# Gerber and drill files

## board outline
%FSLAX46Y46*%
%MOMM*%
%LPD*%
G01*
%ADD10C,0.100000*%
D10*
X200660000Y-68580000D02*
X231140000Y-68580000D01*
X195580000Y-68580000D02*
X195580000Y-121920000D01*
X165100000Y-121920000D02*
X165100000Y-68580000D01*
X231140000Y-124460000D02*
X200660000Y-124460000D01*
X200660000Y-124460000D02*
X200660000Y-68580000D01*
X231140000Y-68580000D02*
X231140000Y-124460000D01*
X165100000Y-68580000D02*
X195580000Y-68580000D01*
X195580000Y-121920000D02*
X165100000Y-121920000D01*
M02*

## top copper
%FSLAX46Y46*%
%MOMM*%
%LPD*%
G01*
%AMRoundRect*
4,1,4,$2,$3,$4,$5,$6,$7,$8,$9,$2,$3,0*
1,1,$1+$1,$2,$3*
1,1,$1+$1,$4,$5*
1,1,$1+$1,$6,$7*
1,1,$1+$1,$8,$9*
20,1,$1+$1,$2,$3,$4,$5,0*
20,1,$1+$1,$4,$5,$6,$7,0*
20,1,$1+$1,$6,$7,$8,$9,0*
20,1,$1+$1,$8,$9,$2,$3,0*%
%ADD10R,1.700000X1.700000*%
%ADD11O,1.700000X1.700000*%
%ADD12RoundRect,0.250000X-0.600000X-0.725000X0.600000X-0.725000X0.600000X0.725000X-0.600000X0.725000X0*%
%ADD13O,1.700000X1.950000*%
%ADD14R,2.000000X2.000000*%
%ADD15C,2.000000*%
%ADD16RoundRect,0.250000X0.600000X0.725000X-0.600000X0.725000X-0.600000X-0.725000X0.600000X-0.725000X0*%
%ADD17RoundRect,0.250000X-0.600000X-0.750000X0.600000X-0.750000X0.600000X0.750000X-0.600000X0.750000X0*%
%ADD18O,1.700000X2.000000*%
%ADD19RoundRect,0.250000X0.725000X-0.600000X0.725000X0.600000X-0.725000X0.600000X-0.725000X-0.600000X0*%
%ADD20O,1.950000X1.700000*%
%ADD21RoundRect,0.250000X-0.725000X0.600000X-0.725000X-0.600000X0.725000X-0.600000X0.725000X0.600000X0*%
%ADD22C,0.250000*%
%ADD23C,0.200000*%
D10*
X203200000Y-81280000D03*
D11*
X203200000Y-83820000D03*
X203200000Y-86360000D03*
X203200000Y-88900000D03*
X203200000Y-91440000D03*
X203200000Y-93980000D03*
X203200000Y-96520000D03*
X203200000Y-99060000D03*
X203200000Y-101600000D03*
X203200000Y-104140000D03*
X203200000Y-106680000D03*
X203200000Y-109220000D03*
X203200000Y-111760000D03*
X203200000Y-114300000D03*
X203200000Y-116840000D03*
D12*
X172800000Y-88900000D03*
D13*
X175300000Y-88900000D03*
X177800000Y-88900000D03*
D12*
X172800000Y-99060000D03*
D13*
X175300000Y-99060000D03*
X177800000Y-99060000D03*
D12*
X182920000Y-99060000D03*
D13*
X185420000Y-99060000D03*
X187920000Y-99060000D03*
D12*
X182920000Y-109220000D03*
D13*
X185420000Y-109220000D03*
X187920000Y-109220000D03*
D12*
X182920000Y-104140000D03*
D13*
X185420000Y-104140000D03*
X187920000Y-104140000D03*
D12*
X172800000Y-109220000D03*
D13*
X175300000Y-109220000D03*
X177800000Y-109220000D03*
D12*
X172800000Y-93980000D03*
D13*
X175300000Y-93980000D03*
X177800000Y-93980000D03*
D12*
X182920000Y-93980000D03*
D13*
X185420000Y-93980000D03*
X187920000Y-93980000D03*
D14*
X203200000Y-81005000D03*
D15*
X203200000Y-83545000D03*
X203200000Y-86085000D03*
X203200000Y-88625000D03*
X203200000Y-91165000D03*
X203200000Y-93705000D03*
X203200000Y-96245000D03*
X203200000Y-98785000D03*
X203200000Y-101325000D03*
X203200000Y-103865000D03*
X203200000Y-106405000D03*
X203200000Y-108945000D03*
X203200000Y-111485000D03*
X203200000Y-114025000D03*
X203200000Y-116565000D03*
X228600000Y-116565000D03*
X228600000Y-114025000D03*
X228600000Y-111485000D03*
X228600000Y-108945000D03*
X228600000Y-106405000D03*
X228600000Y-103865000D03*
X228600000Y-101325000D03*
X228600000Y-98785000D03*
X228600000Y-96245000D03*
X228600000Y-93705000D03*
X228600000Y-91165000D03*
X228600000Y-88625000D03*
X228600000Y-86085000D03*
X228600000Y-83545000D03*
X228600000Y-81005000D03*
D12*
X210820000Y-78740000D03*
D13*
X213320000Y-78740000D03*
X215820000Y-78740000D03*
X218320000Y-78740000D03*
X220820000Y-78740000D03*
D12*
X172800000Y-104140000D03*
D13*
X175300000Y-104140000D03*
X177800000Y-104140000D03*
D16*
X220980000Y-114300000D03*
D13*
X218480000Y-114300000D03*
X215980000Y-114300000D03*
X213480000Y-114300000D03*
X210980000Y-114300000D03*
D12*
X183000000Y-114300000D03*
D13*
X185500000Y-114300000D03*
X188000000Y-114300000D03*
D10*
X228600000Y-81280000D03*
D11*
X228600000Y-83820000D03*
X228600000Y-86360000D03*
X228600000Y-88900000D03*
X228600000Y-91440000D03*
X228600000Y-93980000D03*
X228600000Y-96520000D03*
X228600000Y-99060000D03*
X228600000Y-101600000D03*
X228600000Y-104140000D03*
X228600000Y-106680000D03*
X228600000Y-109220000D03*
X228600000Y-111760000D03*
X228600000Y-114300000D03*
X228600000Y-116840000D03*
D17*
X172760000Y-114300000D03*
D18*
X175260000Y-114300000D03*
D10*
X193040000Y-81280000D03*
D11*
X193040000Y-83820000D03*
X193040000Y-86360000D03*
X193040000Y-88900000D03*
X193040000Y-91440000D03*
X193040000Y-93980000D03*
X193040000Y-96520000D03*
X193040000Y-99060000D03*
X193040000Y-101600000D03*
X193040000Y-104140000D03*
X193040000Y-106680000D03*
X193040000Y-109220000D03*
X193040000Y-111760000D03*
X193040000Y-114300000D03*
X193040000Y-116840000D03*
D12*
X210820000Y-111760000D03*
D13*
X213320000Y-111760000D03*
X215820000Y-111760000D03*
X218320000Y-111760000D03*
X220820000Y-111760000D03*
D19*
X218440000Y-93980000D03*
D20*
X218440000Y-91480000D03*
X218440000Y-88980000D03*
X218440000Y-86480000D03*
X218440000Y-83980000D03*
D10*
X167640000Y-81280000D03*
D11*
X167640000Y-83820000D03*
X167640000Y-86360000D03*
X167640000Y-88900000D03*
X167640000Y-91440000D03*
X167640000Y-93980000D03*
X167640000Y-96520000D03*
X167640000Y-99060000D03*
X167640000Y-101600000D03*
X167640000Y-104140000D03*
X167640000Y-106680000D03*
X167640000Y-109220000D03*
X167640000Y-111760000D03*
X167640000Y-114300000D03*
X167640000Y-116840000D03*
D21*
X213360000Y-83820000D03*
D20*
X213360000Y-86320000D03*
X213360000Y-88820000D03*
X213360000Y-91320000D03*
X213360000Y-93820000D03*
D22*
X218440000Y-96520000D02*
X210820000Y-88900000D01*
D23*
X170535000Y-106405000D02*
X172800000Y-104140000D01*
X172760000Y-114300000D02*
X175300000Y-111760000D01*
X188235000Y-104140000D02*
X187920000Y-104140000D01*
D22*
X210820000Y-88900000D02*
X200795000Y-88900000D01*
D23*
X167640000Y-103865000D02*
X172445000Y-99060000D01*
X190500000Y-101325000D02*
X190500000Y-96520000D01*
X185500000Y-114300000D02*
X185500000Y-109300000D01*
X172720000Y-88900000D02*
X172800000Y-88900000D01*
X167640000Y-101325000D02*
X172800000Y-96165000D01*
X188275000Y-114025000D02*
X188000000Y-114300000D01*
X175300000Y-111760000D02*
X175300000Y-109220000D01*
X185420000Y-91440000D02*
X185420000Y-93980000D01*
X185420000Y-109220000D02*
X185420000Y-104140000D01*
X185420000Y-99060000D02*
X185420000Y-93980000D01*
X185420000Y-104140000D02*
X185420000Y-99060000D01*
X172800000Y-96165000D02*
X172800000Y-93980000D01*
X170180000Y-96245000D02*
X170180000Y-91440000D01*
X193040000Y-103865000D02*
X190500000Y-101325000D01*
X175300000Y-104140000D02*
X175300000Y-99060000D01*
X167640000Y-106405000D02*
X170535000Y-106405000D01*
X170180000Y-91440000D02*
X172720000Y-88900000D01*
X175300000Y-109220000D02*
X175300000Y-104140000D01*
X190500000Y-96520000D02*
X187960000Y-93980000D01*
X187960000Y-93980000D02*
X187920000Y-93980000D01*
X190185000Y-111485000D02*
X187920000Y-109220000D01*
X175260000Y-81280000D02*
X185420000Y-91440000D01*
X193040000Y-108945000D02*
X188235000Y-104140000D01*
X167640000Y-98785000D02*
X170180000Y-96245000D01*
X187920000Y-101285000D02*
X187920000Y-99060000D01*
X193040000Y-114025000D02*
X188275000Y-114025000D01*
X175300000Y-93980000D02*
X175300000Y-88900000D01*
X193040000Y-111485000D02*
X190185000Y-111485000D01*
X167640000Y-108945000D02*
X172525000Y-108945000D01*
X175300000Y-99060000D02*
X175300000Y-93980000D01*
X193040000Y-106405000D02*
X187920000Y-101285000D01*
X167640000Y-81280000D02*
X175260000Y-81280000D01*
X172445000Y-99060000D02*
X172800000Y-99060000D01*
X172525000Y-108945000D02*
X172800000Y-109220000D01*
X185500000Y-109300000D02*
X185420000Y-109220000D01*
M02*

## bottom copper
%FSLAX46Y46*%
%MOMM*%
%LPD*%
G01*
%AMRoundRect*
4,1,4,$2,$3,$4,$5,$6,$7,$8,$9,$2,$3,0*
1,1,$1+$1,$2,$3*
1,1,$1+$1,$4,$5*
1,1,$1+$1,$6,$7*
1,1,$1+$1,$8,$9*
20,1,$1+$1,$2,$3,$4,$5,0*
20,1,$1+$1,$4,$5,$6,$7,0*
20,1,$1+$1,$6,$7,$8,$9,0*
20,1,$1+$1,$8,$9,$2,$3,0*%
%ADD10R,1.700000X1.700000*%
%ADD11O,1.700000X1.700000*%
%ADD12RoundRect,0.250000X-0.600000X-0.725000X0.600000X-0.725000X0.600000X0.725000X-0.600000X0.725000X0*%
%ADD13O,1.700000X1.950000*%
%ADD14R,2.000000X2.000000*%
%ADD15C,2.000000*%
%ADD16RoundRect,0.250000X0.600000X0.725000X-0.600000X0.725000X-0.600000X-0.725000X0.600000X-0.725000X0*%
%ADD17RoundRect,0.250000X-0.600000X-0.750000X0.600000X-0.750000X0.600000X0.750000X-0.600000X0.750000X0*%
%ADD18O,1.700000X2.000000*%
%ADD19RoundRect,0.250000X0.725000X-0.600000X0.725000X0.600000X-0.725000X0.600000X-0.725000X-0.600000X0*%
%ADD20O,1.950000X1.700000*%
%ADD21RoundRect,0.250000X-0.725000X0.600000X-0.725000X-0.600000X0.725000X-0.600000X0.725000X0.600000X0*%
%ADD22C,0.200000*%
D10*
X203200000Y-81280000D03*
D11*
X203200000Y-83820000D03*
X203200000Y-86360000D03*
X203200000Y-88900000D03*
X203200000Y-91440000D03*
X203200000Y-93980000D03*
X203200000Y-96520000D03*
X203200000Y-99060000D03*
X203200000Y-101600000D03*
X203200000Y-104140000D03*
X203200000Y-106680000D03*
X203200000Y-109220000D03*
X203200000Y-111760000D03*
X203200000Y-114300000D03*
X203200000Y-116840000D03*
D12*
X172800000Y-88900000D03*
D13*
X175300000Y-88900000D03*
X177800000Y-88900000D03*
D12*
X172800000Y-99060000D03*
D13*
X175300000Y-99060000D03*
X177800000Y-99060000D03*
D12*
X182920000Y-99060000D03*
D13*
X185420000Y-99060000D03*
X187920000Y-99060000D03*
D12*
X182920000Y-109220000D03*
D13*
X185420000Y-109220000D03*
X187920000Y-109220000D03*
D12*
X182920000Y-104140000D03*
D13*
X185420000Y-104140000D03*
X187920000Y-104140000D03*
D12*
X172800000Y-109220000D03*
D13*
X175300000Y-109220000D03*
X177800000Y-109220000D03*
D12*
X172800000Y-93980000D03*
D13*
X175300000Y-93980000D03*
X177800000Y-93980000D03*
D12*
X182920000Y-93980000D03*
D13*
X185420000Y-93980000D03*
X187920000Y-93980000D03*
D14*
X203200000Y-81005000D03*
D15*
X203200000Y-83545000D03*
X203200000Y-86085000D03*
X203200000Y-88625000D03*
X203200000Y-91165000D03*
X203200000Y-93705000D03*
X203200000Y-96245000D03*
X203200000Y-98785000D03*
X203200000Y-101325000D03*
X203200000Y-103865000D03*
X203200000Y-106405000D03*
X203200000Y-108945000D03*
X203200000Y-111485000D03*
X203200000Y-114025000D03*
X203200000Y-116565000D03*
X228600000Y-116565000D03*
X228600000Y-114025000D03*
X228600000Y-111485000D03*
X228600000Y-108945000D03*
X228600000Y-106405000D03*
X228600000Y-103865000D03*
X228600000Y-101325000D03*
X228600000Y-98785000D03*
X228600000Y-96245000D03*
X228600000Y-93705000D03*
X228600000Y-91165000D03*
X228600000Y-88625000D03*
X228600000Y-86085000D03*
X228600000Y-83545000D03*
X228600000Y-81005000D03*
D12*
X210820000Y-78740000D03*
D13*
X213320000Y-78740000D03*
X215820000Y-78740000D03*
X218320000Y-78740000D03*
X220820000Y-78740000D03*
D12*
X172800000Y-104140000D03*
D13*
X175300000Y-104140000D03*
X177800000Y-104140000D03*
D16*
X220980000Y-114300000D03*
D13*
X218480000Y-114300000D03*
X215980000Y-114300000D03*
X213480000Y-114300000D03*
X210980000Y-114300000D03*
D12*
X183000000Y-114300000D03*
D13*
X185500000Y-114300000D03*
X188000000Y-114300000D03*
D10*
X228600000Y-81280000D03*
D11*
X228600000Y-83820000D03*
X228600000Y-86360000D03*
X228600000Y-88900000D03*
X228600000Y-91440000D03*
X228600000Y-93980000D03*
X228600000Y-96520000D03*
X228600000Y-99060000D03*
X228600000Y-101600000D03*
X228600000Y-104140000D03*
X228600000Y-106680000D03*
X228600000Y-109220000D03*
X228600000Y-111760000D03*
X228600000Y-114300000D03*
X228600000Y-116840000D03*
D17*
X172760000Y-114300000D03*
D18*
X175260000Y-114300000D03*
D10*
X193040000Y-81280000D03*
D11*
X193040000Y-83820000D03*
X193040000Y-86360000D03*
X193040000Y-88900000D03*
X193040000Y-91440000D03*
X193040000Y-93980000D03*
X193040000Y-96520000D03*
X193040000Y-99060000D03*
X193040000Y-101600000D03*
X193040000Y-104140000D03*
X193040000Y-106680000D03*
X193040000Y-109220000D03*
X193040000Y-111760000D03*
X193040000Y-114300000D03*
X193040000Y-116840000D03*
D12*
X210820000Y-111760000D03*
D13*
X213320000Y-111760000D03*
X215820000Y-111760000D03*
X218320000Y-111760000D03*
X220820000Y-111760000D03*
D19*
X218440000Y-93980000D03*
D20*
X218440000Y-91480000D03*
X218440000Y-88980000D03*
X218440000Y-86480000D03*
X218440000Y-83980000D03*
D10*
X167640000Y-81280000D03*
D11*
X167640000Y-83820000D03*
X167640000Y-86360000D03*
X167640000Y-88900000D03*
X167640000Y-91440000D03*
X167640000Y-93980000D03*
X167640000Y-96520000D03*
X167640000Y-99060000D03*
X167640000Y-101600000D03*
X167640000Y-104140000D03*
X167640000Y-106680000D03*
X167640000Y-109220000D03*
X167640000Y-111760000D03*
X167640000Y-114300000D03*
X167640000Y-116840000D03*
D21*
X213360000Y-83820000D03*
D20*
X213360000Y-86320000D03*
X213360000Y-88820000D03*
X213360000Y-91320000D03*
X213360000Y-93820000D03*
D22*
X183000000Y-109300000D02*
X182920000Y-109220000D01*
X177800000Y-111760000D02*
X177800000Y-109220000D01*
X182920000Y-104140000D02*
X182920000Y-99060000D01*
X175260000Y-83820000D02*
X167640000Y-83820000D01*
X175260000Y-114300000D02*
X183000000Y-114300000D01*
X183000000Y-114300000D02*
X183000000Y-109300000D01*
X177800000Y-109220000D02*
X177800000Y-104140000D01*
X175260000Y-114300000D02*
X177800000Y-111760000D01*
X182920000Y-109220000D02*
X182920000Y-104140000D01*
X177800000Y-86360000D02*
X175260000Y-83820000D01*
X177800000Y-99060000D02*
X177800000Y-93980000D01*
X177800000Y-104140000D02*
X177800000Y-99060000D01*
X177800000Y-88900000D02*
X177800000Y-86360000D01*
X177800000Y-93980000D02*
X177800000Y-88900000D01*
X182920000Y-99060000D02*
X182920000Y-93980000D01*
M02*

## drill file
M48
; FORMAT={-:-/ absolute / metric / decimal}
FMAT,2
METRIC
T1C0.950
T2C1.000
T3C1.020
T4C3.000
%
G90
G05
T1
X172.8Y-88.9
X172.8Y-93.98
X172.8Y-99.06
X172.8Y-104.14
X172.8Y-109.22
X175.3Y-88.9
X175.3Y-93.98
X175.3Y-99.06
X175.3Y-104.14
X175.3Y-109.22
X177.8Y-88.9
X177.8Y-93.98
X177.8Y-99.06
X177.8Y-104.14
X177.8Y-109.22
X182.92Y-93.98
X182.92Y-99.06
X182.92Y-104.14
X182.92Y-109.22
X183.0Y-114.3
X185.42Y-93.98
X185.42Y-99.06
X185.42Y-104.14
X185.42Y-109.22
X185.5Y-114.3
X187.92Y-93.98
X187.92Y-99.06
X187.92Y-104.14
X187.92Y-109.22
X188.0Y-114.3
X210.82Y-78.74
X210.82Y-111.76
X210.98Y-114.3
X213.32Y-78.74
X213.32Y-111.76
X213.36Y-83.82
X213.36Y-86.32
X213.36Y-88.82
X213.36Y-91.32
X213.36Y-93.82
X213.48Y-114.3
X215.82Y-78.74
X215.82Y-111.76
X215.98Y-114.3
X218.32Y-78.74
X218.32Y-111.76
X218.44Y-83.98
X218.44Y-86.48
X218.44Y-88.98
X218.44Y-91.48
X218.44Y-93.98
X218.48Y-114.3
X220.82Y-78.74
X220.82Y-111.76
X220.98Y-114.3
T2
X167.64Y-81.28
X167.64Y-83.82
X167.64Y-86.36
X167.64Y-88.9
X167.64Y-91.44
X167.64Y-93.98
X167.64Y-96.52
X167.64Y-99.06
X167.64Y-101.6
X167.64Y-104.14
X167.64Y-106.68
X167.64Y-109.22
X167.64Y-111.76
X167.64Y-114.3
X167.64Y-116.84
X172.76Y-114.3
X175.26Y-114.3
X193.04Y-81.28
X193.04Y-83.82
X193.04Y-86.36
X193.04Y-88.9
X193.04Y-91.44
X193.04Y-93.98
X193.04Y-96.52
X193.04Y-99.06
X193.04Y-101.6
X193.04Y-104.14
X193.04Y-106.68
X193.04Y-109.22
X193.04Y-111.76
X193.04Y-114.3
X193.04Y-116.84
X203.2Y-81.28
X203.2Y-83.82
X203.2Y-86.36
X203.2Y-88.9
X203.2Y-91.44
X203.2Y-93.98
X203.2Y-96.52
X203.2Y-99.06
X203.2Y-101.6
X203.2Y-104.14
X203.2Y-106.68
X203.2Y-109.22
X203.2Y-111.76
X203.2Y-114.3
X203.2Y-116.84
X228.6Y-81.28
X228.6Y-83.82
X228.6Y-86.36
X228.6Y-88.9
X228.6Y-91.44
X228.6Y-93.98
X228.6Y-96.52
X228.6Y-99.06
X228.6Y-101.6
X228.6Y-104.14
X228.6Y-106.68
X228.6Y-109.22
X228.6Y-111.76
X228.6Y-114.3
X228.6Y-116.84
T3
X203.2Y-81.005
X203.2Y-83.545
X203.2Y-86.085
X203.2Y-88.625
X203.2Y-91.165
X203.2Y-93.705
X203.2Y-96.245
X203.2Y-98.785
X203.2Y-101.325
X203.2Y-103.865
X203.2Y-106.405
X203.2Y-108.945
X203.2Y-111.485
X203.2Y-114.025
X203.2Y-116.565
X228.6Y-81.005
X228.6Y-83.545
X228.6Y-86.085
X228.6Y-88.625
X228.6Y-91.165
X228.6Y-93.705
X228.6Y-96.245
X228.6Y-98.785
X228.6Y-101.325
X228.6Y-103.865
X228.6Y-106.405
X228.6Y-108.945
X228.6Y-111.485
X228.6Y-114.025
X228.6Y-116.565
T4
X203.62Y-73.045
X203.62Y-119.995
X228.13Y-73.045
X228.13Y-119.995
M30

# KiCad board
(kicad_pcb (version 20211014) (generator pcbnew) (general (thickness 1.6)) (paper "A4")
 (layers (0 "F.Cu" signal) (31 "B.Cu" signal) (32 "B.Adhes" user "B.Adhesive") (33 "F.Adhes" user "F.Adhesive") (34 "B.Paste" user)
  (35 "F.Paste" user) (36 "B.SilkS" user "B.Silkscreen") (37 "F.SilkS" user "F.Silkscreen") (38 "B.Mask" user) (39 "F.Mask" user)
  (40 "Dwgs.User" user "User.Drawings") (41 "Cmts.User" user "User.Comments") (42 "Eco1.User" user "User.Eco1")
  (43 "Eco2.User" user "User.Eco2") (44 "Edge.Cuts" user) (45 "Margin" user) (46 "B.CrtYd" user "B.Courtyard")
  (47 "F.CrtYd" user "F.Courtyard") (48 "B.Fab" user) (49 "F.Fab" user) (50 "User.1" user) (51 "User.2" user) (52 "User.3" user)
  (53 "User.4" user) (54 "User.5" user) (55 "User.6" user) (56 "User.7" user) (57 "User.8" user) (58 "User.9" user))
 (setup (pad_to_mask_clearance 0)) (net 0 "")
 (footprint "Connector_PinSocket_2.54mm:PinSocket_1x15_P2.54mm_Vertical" (layer "F.Cu") (at 203.2 81.28)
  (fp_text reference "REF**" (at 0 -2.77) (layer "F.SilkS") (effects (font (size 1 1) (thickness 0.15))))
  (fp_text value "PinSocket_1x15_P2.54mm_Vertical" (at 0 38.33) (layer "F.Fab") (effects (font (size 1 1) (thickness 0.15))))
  (pad "1" thru_hole rect (at 0 0) (size 1.7 1.7) (drill 1) (layers *.Cu *.Mask))
  (pad "2" thru_hole oval (at 0 2.54) (size 1.7 1.7) (drill 1) (layers *.Cu *.Mask))
  (pad "3" thru_hole oval (at 0 5.08) (size 1.7 1.7) (drill 1) (layers *.Cu *.Mask))
  (pad "4" thru_hole oval (at 0 7.62) (size 1.7 1.7) (drill 1) (layers *.Cu *.Mask))
  (pad "5" thru_hole oval (at 0 10.16) (size 1.7 1.7) (drill 1) (layers *.Cu *.Mask))
  (pad "6" thru_hole oval (at 0 12.7) (size 1.7 1.7) (drill 1) (layers *.Cu *.Mask))
  (pad "7" thru_hole oval (at 0 15.24) (size 1.7 1.7) (drill 1) (layers *.Cu *.Mask))
  (pad "8" thru_hole oval (at 0 17.78) (size 1.7 1.7) (drill 1) (layers *.Cu *.Mask))
  (pad "9" thru_hole oval (at 0 20.32) (size 1.7 1.7) (drill 1) (layers *.Cu *.Mask))
  (pad "10" thru_hole oval (at 0 22.86) (size 1.7 1.7) (drill 1) (layers *.Cu *.Mask))
  (pad "11" thru_hole oval (at 0 25.4) (size 1.7 1.7) (drill 1) (layers *.Cu *.Mask))
  (pad "12" thru_hole oval (at 0 27.94) (size 1.7 1.7) (drill 1) (layers *.Cu *.Mask))
  (pad "13" thru_hole oval (at 0 30.48) (size 1.7 1.7) (drill 1) (layers *.Cu *.Mask))
  (pad "14" thru_hole oval (at 0 33.02) (size 1.7 1.7) (drill 1) (layers *.Cu *.Mask))
  (pad "15" thru_hole oval (at 0 35.56) (size 1.7 1.7) (drill 1) (layers *.Cu *.Mask)))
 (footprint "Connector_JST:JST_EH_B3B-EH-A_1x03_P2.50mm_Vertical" (layer "F.Cu") (at 172.8 88.9)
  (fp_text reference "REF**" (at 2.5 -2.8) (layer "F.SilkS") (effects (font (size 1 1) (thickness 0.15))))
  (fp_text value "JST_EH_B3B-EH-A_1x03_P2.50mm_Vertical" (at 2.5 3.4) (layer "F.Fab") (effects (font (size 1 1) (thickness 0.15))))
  (pad "1" thru_hole roundrect (at 0 0) (size 1.7 1.95) (drill 0.95) (layers *.Cu *.Mask) (roundrect_rratio 0.147059))
  (pad "2" thru_hole oval (at 2.5 0) (size 1.7 1.95) (drill 0.95) (layers *.Cu *.Mask))
  (pad "3" thru_hole oval (at 5 0) (size 1.7 1.95) (drill 0.95) (layers *.Cu *.Mask)))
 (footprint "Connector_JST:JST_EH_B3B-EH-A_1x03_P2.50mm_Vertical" (layer "F.Cu") (at 172.8 99.06)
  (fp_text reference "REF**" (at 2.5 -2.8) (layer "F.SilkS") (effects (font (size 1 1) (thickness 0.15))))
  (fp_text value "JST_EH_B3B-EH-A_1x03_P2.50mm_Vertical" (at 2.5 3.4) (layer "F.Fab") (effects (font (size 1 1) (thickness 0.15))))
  (pad "1" thru_hole roundrect (at 0 0) (size 1.7 1.95) (drill 0.95) (layers *.Cu *.Mask) (roundrect_rratio 0.147059))
  (pad "2" thru_hole oval (at 2.5 0) (size 1.7 1.95) (drill 0.95) (layers *.Cu *.Mask))
  (pad "3" thru_hole oval (at 5 0) (size 1.7 1.95) (drill 0.95) (layers *.Cu *.Mask)))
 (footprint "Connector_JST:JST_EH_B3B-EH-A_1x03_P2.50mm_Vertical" (layer "F.Cu") (at 182.92 99.06)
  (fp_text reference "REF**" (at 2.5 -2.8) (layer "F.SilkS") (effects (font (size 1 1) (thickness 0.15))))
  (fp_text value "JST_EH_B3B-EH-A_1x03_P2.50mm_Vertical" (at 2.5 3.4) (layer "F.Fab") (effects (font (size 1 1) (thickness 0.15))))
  (pad "1" thru_hole roundrect (at 0 0) (size 1.7 1.95) (drill 0.95) (layers *.Cu *.Mask) (roundrect_rratio 0.147059))
  (pad "2" thru_hole oval (at 2.5 0) (size 1.7 1.95) (drill 0.95) (layers *.Cu *.Mask))
  (pad "3" thru_hole oval (at 5 0) (size 1.7 1.95) (drill 0.95) (layers *.Cu *.Mask)))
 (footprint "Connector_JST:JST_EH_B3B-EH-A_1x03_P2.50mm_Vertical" (layer "F.Cu") (at 182.92 109.22)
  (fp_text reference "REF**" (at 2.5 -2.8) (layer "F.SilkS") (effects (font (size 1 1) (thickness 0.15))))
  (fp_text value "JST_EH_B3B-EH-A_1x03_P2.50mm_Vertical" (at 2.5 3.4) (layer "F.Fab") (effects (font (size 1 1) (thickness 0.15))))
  (pad "1" thru_hole roundrect (at 0 0) (size 1.7 1.95) (drill 0.95) (layers *.Cu *.Mask) (roundrect_rratio 0.147059))
  (pad "2" thru_hole oval (at 2.5 0) (size 1.7 1.95) (drill 0.95) (layers *.Cu *.Mask))
  (pad "3" thru_hole oval (at 5 0) (size 1.7 1.95) (drill 0.95) (layers *.Cu *.Mask)))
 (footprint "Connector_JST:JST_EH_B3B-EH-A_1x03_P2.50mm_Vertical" (layer "F.Cu") (at 182.92 104.14)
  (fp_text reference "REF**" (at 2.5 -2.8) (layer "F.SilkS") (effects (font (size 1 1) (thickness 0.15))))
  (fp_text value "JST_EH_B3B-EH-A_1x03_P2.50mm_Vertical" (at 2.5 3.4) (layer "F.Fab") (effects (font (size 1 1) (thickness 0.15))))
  (pad "1" thru_hole roundrect (at 0 0) (size 1.7 1.95) (drill 0.95) (layers *.Cu *.Mask) (roundrect_rratio 0.147059))
  (pad "2" thru_hole oval (at 2.5 0) (size 1.7 1.95) (drill 0.95) (layers *.Cu *.Mask))
  (pad "3" thru_hole oval (at 5 0) (size 1.7 1.95) (drill 0.95) (layers *.Cu *.Mask)))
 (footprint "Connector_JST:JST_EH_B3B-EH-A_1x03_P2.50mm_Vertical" (layer "F.Cu") (at 172.8 109.22)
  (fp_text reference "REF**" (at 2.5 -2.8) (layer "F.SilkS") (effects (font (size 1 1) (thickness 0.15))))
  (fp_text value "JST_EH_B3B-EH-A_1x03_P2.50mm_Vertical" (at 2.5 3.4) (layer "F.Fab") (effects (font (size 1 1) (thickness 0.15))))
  (pad "1" thru_hole roundrect (at 0 0) (size 1.7 1.95) (drill 0.95) (layers *.Cu *.Mask) (roundrect_rratio 0.147059))
  (pad "2" thru_hole oval (at 2.5 0) (size 1.7 1.95) (drill 0.95) (layers *.Cu *.Mask))
  (pad "3" thru_hole oval (at 5 0) (size 1.7 1.95) (drill 0.95) (layers *.Cu *.Mask)))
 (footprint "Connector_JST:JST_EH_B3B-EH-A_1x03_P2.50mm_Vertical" (layer "F.Cu") (at 172.8 93.98)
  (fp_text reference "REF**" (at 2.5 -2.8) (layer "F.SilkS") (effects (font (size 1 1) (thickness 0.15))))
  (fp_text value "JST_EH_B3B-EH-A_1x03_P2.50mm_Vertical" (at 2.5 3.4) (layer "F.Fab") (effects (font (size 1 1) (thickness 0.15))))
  (pad "1" thru_hole roundrect (at 0 0) (size 1.7 1.95) (drill 0.95) (layers *.Cu *.Mask) (roundrect_rratio 0.147059))
  (pad "2" thru_hole oval (at 2.5 0) (size 1.7 1.95) (drill 0.95) (layers *.Cu *.Mask))
  (pad "3" thru_hole oval (at 5 0) (size 1.7 1.95) (drill 0.95) (layers *.Cu *.Mask)))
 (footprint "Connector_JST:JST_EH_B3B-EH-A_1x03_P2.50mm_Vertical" (layer "F.Cu") (at 182.92 93.98)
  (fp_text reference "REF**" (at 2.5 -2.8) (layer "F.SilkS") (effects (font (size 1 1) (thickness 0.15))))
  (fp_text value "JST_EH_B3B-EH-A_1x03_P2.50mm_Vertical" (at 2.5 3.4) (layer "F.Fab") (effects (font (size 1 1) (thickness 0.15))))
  (pad "1" thru_hole roundrect (at 0 0) (size 1.7 1.95) (drill 0.95) (layers *.Cu *.Mask) (roundrect_rratio 0.147059))
  (pad "2" thru_hole oval (at 2.5 0) (size 1.7 1.95) (drill 0.95) (layers *.Cu *.Mask))
  (pad "3" thru_hole oval (at 5 0) (size 1.7 1.95) (drill 0.95) (layers *.Cu *.Mask)))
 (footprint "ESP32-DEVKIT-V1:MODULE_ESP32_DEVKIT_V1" (layer "F.Cu") (at 215.9 96.52)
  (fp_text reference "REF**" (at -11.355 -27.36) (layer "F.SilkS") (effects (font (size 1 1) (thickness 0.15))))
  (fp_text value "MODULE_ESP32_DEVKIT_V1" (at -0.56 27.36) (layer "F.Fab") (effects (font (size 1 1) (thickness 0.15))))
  (pad "" np_thru_hole circle (at -12.28 23.475) (size 3 3) (drill 3) (layers *.Cu *.Mask))
  (pad "" np_thru_hole circle (at -12.28 -23.475) (size 3 3) (drill 3) (layers *.Cu *.Mask))
  (pad "" np_thru_hole circle (at 12.23 23.475) (size 3 3) (drill 3) (layers *.Cu *.Mask))
  (pad "" np_thru_hole circle (at 12.23 -23.475) (size 3 3) (drill 3) (layers *.Cu *.Mask))
  (pad "1" thru_hole rect (at -12.7 -15.515) (size 2 2) (drill 1.02) (layers *.Cu *.Mask))
  (pad "2" thru_hole circle (at -12.7 -12.975) (size 2 2) (drill 1.02) (layers *.Cu *.Mask))
  (pad "3" thru_hole circle (at -12.7 -10.435) (size 2 2) (drill 1.02) (layers *.Cu *.Mask))
  (pad "4" thru_hole circle (at -12.7 -7.895) (size 2 2) (drill 1.02) (layers *.Cu *.Mask))
  (pad "5" thru_hole circle (at -12.7 -5.355) (size 2 2) (drill 1.02) (layers *.Cu *.Mask))
  (pad "6" thru_hole circle (at -12.7 -2.815) (size 2 2) (drill 1.02) (layers *.Cu *.Mask))
  (pad "7" thru_hole circle (at -12.7 -0.275) (size 2 2) (drill 1.02) (layers *.Cu *.Mask))
  (pad "8" thru_hole circle (at -12.7 2.265) (size 2 2) (drill 1.02) (layers *.Cu *.Mask))
  (pad "9" thru_hole circle (at -12.7 4.805) (size 2 2) (drill 1.02) (layers *.Cu *.Mask))
  (pad "10" thru_hole circle (at -12.7 7.345) (size 2 2) (drill 1.02) (layers *.Cu *.Mask))
  (pad "11" thru_hole circle (at -12.7 9.885) (size 2 2) (drill 1.02) (layers *.Cu *.Mask))
  (pad "12" thru_hole circle (at -12.7 12.425) (size 2 2) (drill 1.02) (layers *.Cu *.Mask))
  (pad "13" thru_hole circle (at -12.7 14.965) (size 2 2) (drill 1.02) (layers *.Cu *.Mask))
  (pad "14" thru_hole circle (at -12.7 17.505) (size 2 2) (drill 1.02) (layers *.Cu *.Mask))
  (pad "15" thru_hole circle (at -12.7 20.045) (size 2 2) (drill 1.02) (layers *.Cu *.Mask))
  (pad "16" thru_hole circle (at 12.7 20.045) (size 2 2) (drill 1.02) (layers *.Cu *.Mask))
  (pad "17" thru_hole circle (at 12.7 17.505) (size 2 2) (drill 1.02) (layers *.Cu *.Mask))
  (pad "18" thru_hole circle (at 12.7 14.965) (size 2 2) (drill 1.02) (layers *.Cu *.Mask))
  (pad "19" thru_hole circle (at 12.7 12.425) (size 2 2) (drill 1.02) (layers *.Cu *.Mask))
  (pad "20" thru_hole circle (at 12.7 9.885) (size 2 2) (drill 1.02) (layers *.Cu *.Mask))
  (pad "21" thru_hole circle (at 12.7 7.345) (size 2 2) (drill 1.02) (layers *.Cu *.Mask))
  (pad "22" thru_hole circle (at 12.7 4.805) (size 2 2) (drill 1.02) (layers *.Cu *.Mask))
  (pad "23" thru_hole circle (at 12.7 2.265) (size 2 2) (drill 1.02) (layers *.Cu *.Mask))
  (pad "24" thru_hole circle (at 12.7 -0.275) (size 2 2) (drill 1.02) (layers *.Cu *.Mask))
  (pad "25" thru_hole circle (at 12.7 -2.815) (size 2 2) (drill 1.02) (layers *.Cu *.Mask))
  (pad "26" thru_hole circle (at 12.7 -5.355) (size 2 2) (drill 1.02) (layers *.Cu *.Mask))
  (pad "27" thru_hole circle (at 12.7 -7.895) (size 2 2) (drill 1.02) (layers *.Cu *.Mask))
  (pad "28" thru_hole circle (at 12.7 -10.435) (size 2 2) (drill 1.02) (layers *.Cu *.Mask))
  (pad "29" thru_hole circle (at 12.7 -12.975) (size 2 2) (drill 1.02) (layers *.Cu *.Mask))
  (pad "30" thru_hole circle (at 12.7 -15.515) (size 2 2) (drill 1.02) (layers *.Cu *.Mask))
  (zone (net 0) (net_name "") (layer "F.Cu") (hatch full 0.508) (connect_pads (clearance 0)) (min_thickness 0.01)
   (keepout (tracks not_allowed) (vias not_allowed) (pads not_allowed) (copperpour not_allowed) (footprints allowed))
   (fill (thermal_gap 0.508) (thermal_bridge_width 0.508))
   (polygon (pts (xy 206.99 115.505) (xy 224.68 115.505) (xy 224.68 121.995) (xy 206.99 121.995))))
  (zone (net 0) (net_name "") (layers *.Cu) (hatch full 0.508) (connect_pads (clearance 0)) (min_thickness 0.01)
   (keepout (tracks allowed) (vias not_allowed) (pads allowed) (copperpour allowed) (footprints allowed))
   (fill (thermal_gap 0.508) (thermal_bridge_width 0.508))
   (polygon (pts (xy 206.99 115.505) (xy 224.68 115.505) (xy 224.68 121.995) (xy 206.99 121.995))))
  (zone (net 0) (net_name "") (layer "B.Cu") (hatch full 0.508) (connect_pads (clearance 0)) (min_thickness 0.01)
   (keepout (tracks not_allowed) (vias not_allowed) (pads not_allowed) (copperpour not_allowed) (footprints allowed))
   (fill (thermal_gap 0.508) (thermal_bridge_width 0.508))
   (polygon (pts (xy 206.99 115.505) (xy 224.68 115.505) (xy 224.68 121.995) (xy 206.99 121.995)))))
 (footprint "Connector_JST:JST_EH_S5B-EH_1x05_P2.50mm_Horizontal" (layer "F.Cu") (at 210.82 78.74)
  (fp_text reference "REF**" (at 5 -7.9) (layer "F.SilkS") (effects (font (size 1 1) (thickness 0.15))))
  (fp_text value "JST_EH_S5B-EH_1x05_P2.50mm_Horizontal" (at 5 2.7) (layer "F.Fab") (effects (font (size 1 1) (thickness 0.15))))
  (pad "1" thru_hole roundrect (at 0 0) (size 1.7 1.95) (drill 0.95) (layers *.Cu *.Mask) (roundrect_rratio 0.147059))
  (pad "2" thru_hole oval (at 2.5 0) (size 1.7 1.95) (drill 0.95) (layers *.Cu *.Mask))
  (pad "3" thru_hole oval (at 5 0) (size 1.7 1.95) (drill 0.95) (layers *.Cu *.Mask))
  (pad "4" thru_hole oval (at 7.5 0) (size 1.7 1.95) (drill 0.95) (layers *.Cu *.Mask))
  (pad "5" thru_hole oval (at 10 0) (size 1.7 1.95) (drill 0.95) (layers *.Cu *.Mask)))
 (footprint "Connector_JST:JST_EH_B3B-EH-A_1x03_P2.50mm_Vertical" (layer "F.Cu") (at 172.8 104.14)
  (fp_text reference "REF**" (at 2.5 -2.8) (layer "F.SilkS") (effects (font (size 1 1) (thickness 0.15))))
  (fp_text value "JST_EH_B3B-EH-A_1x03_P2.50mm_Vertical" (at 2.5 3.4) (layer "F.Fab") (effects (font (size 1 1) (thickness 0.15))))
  (pad "1" thru_hole roundrect (at 0 0) (size 1.7 1.95) (drill 0.95) (layers *.Cu *.Mask) (roundrect_rratio 0.147059))
  (pad "2" thru_hole oval (at 2.5 0) (size 1.7 1.95) (drill 0.95) (layers *.Cu *.Mask))
  (pad "3" thru_hole oval (at 5 0) (size 1.7 1.95) (drill 0.95) (layers *.Cu *.Mask)))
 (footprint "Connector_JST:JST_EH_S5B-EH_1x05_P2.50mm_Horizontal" (layer "F.Cu") (at 220.98 114.3 180)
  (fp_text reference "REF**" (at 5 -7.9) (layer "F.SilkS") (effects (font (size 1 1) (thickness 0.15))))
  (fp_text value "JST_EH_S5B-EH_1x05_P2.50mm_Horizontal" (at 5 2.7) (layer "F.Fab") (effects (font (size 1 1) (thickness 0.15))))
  (pad "1" thru_hole roundrect (at 0 0 180) (size 1.7 1.95) (drill 0.95) (layers *.Cu *.Mask) (roundrect_rratio 0.147059))
  (pad "2" thru_hole oval (at 2.5 0 180) (size 1.7 1.95) (drill 0.95) (layers *.Cu *.Mask))
  (pad "3" thru_hole oval (at 5 0 180) (size 1.7 1.95) (drill 0.95) (layers *.Cu *.Mask))
  (pad "4" thru_hole oval (at 7.5 0 180) (size 1.7 1.95) (drill 0.95) (layers *.Cu *.Mask))
  (pad "5" thru_hole oval (at 10 0 180) (size 1.7 1.95) (drill 0.95) (layers *.Cu *.Mask)))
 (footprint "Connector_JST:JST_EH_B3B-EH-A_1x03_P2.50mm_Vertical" (layer "F.Cu") (at 183 114.3)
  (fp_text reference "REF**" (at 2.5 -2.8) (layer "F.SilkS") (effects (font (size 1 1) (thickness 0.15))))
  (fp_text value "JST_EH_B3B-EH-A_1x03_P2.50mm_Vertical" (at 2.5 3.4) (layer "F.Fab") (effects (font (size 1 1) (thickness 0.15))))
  (pad "1" thru_hole roundrect (at 0 0) (size 1.7 1.95) (drill 0.95) (layers *.Cu *.Mask) (roundrect_rratio 0.147059))
  (pad "2" thru_hole oval (at 2.5 0) (size 1.7 1.95) (drill 0.95) (layers *.Cu *.Mask))
  (pad "3" thru_hole oval (at 5 0) (size 1.7 1.95) (drill 0.95) (layers *.Cu *.Mask)))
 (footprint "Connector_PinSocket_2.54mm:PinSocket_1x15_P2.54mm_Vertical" (layer "F.Cu") (at 228.6 81.28)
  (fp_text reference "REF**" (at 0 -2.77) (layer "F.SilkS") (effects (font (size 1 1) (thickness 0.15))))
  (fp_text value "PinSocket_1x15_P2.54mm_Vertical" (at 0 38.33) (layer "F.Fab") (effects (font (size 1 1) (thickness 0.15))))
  (pad "1" thru_hole rect (at 0 0) (size 1.7 1.7) (drill 1) (layers *.Cu *.Mask))
  (pad "2" thru_hole oval (at 0 2.54) (size 1.7 1.7) (drill 1) (layers *.Cu *.Mask))
  (pad "3" thru_hole oval (at 0 5.08) (size 1.7 1.7) (drill 1) (layers *.Cu *.Mask))
  (pad "4" thru_hole oval (at 0 7.62) (size 1.7 1.7) (drill 1) (layers *.Cu *.Mask))
  (pad "5" thru_hole oval (at 0 10.16) (size 1.7 1.7) (drill 1) (layers *.Cu *.Mask))
  (pad "6" thru_hole oval (at 0 12.7) (size 1.7 1.7) (drill 1) (layers *.Cu *.Mask))
  (pad "7" thru_hole oval (at 0 15.24) (size 1.7 1.7) (drill 1) (layers *.Cu *.Mask))
  (pad "8" thru_hole oval (at 0 17.78) (size 1.7 1.7) (drill 1) (layers *.Cu *.Mask))
  (pad "9" thru_hole oval (at 0 20.32) (size 1.7 1.7) (drill 1) (layers *.Cu *.Mask))
  (pad "10" thru_hole oval (at 0 22.86) (size 1.7 1.7) (drill 1) (layers *.Cu *.Mask))
  (pad "11" thru_hole oval (at 0 25.4) (size 1.7 1.7) (drill 1) (layers *.Cu *.Mask))
  (pad "12" thru_hole oval (at 0 27.94) (size 1.7 1.7) (drill 1) (layers *.Cu *.Mask))
  (pad "13" thru_hole oval (at 0 30.48) (size 1.7 1.7) (drill 1) (layers *.Cu *.Mask))
  (pad "14" thru_hole oval (at 0 33.02) (size 1.7 1.7) (drill 1) (layers *.Cu *.Mask))
  (pad "15" thru_hole oval (at 0 35.56) (size 1.7 1.7) (drill 1) (layers *.Cu *.Mask)))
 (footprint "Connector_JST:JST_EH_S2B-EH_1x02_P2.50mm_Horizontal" (layer "B.Cu") (at 172.76 114.3)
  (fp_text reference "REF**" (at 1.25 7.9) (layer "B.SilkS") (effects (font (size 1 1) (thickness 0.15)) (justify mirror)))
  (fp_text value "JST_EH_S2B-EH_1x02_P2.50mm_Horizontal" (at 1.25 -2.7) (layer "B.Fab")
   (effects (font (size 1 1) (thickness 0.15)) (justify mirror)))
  (pad "1" thru_hole roundrect (at 0 0) (size 1.7 2) (drill 1) (layers *.Cu *.Mask) (roundrect_rratio 0.147059))
  (pad "2" thru_hole oval (at 2.5 0) (size 1.7 2) (drill 1) (layers *.Cu *.Mask)))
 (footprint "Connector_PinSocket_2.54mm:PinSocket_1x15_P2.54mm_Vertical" (layer "B.Cu") (at 193.04 81.28 180)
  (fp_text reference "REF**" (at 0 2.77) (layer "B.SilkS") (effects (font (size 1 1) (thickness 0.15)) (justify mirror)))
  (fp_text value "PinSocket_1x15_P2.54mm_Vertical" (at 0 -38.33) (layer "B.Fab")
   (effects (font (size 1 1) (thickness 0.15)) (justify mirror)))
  (pad "1" thru_hole rect (at 0 0 180) (size 1.7 1.7) (drill 1) (layers *.Cu *.Mask))
  (pad "2" thru_hole oval (at 0 -2.54 180) (size 1.7 1.7) (drill 1) (layers *.Cu *.Mask))
  (pad "3" thru_hole oval (at 0 -5.08 180) (size 1.7 1.7) (drill 1) (layers *.Cu *.Mask))
  (pad "4" thru_hole oval (at 0 -7.62 180) (size 1.7 1.7) (drill 1) (layers *.Cu *.Mask))
  (pad "5" thru_hole oval (at 0 -10.16 180) (size 1.7 1.7) (drill 1) (layers *.Cu *.Mask))
  (pad "6" thru_hole oval (at 0 -12.7 180) (size 1.7 1.7) (drill 1) (layers *.Cu *.Mask))
  (pad "7" thru_hole oval (at 0 -15.24 180) (size 1.7 1.7) (drill 1) (layers *.Cu *.Mask))
  (pad "8" thru_hole oval (at 0 -17.78 180) (size 1.7 1.7) (drill 1) (layers *.Cu *.Mask))
  (pad "9" thru_hole oval (at 0 -20.32 180) (size 1.7 1.7) (drill 1) (layers *.Cu *.Mask))
  (pad "10" thru_hole oval (at 0 -22.86 180) (size 1.7 1.7) (drill 1) (layers *.Cu *.Mask))
  (pad "11" thru_hole oval (at 0 -25.4 180) (size 1.7 1.7) (drill 1) (layers *.Cu *.Mask))
  (pad "12" thru_hole oval (at 0 -27.94 180) (size 1.7 1.7) (drill 1) (layers *.Cu *.Mask))
  (pad "13" thru_hole oval (at 0 -30.48 180) (size 1.7 1.7) (drill 1) (layers *.Cu *.Mask))
  (pad "14" thru_hole oval (at 0 -33.02 180) (size 1.7 1.7) (drill 1) (layers *.Cu *.Mask))
  (pad "15" thru_hole oval (at 0 -35.56 180) (size 1.7 1.7) (drill 1) (layers *.Cu *.Mask)))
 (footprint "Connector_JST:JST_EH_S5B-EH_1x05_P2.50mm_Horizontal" (layer "B.Cu") (at 210.82 111.76)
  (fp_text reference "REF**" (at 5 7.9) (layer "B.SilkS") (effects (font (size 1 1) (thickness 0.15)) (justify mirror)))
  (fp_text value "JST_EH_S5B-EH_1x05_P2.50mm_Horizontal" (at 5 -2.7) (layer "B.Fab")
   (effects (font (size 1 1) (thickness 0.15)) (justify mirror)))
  (pad "1" thru_hole roundrect (at 0 0) (size 1.7 1.95) (drill 0.95) (layers *.Cu *.Mask) (roundrect_rratio 0.147059))
  (pad "2" thru_hole oval (at 2.5 0) (size 1.7 1.95) (drill 0.95) (layers *.Cu *.Mask))
  (pad "3" thru_hole oval (at 5 0) (size 1.7 1.95) (drill 0.95) (layers *.Cu *.Mask))
  (pad "4" thru_hole oval (at 7.5 0) (size 1.7 1.95) (drill 0.95) (layers *.Cu *.Mask))
  (pad "5" thru_hole oval (at 10 0) (size 1.7 1.95) (drill 0.95) (layers *.Cu *.Mask)))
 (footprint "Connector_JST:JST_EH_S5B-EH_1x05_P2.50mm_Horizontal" (layer "B.Cu") (at 218.44 93.98 90)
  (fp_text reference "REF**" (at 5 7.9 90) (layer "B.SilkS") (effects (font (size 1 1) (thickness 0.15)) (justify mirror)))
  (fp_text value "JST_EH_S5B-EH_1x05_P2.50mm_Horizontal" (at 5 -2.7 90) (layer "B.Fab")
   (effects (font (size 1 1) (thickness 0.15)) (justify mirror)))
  (pad "1" thru_hole roundrect (at 0 0 90) (size 1.7 1.95) (drill 0.95) (layers *.Cu *.Mask) (roundrect_rratio 0.147059))
  (pad "2" thru_hole oval (at 2.5 0 90) (size 1.7 1.95) (drill 0.95) (layers *.Cu *.Mask))
  (pad "3" thru_hole oval (at 5 0 90) (size 1.7 1.95) (drill 0.95) (layers *.Cu *.Mask))
  (pad "4" thru_hole oval (at 7.5 0 90) (size 1.7 1.95) (drill 0.95) (layers *.Cu *.Mask))
  (pad "5" thru_hole oval (at 10 0 90) (size 1.7 1.95) (drill 0.95) (layers *.Cu *.Mask)))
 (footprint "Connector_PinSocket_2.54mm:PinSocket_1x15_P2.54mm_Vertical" (layer "B.Cu") (at 167.64 81.28 180)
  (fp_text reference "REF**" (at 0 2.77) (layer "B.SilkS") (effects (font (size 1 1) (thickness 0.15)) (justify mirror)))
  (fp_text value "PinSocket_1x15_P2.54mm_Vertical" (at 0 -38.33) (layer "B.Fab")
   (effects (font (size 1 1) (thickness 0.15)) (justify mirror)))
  (pad "1" thru_hole rect (at 0 0 180) (size 1.7 1.7) (drill 1) (layers *.Cu *.Mask))
  (pad "2" thru_hole oval (at 0 -2.54 180) (size 1.7 1.7) (drill 1) (layers *.Cu *.Mask))
  (pad "3" thru_hole oval (at 0 -5.08 180) (size 1.7 1.7) (drill 1) (layers *.Cu *.Mask))
  (pad "4" thru_hole oval (at 0 -7.62 180) (size 1.7 1.7) (drill 1) (layers *.Cu *.Mask))
  (pad "5" thru_hole oval (at 0 -10.16 180) (size 1.7 1.7) (drill 1) (layers *.Cu *.Mask))
  (pad "6" thru_hole oval (at 0 -12.7 180) (size 1.7 1.7) (drill 1) (layers *.Cu *.Mask))
  (pad "7" thru_hole oval (at 0 -15.24 180) (size 1.7 1.7) (drill 1) (layers *.Cu *.Mask))
  (pad "8" thru_hole oval (at 0 -17.78 180) (size 1.7 1.7) (drill 1) (layers *.Cu *.Mask))
  (pad "9" thru_hole oval (at 0 -20.32 180) (size 1.7 1.7) (drill 1) (layers *.Cu *.Mask))
  (pad "10" thru_hole oval (at 0 -22.86 180) (size 1.7 1.7) (drill 1) (layers *.Cu *.Mask))
  (pad "11" thru_hole oval (at 0 -25.4 180) (size 1.7 1.7) (drill 1) (layers *.Cu *.Mask))
  (pad "12" thru_hole oval (at 0 -27.94 180) (size 1.7 1.7) (drill 1) (layers *.Cu *.Mask))
  (pad "13" thru_hole oval (at 0 -30.48 180) (size 1.7 1.7) (drill 1) (layers *.Cu *.Mask))
  (pad "14" thru_hole oval (at 0 -33.02 180) (size 1.7 1.7) (drill 1) (layers *.Cu *.Mask))
  (pad "15" thru_hole oval (at 0 -35.56 180) (size 1.7 1.7) (drill 1) (layers *.Cu *.Mask)))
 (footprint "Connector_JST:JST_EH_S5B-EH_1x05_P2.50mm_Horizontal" (layer "B.Cu") (at 213.36 83.82 -90)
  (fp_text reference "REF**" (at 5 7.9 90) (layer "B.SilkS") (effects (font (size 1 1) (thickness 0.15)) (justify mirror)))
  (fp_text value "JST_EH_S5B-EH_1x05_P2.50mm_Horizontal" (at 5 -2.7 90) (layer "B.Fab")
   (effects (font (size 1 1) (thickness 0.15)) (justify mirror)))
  (pad "1" thru_hole roundrect (at 0 0 270) (size 1.7 1.95) (drill 0.95) (layers *.Cu *.Mask) (roundrect_rratio 0.147059))
  (pad "2" thru_hole oval (at 2.5 0 270) (size 1.7 1.95) (drill 0.95) (layers *.Cu *.Mask))
  (pad "3" thru_hole oval (at 5 0 270) (size 1.7 1.95) (drill 0.95) (layers *.Cu *.Mask))
  (pad "4" thru_hole oval (at 7.5 0 270) (size 1.7 1.95) (drill 0.95) (layers *.Cu *.Mask))
  (pad "5" thru_hole oval (at 10 0 270) (size 1.7 1.95) (drill 0.95) (layers *.Cu *.Mask)))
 (gr_line (start 200.66 68.58) (end 231.14 68.58) (layer "Edge.Cuts") (width 0.1))
 (gr_line (start 195.58 68.58) (end 195.58 121.92) (layer "Edge.Cuts") (width 0.1))
 (gr_line (start 165.1 121.92) (end 165.1 68.58) (layer "Edge.Cuts") (width 0.1))
 (gr_line (start 231.14 124.46) (end 200.66 124.46) (layer "Edge.Cuts") (width 0.1))
 (gr_line (start 200.66 124.46) (end 200.66 68.58) (layer "Edge.Cuts") (width 0.1))
 (gr_line (start 231.14 68.58) (end 231.14 124.46) (layer "Edge.Cuts") (width 0.1))
 (gr_line (start 165.1 68.58) (end 195.58 68.58) (layer "Edge.Cuts") (width 0.1))
 (gr_line (start 195.58 121.92) (end 165.1 121.92) (layer "Edge.Cuts") (width 0.1))
 (segment (start 218.44 96.52) (end 210.82 88.9) (width 0.25) (layer "F.Cu") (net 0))
 (segment (start 170.535 106.405) (end 172.8 104.14) (width 0.2) (layer "F.Cu") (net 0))
 (segment (start 172.76 114.3) (end 175.3 111.76) (width 0.2) (layer "F.Cu") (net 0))
 (segment (start 188.235 104.14) (end 187.92 104.14) (width 0.2) (layer "F.Cu") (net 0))
 (segment (start 210.82 88.9) (end 200.795 88.9) (width 0.25) (layer "F.Cu") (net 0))
 (segment (start 167.64 103.865) (end 172.445 99.06) (width 0.2) (layer "F.Cu") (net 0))
 (segment (start 190.5 101.325) (end 190.5 96.52) (width 0.2) (layer "F.Cu") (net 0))
 (segment (start 185.5 114.3) (end 185.5 109.3) (width 0.2) (layer "F.Cu") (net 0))
 (segment (start 172.72 88.9) (end 172.8 88.9) (width 0.2) (layer "F.Cu") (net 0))
 (segment (start 167.64 101.325) (end 172.8 96.165) (width 0.2) (layer "F.Cu") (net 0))
 (segment (start 188.275 114.025) (end 188 114.3) (width 0.2) (layer "F.Cu") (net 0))
 (segment (start 175.3 111.76) (end 175.3 109.22) (width 0.2) (layer "F.Cu") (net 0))
 (segment (start 185.42 91.44) (end 185.42 93.98) (width 0.2) (layer "F.Cu") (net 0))
 (segment (start 185.42 109.22) (end 185.42 104.14) (width 0.2) (layer "F.Cu") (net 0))
 (segment (start 185.42 99.06) (end 185.42 93.98) (width 0.2) (layer "F.Cu") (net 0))
 (segment (start 185.42 104.14) (end 185.42 99.06) (width 0.2) (layer "F.Cu") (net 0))
 (segment (start 172.8 96.165) (end 172.8 93.98) (width 0.2) (layer "F.Cu") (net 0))
 (segment (start 170.18 96.245) (end 170.18 91.44) (width 0.2) (layer "F.Cu") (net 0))
 (segment (start 193.04 103.865) (end 190.5 101.325) (width 0.2) (layer "F.Cu") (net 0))
 (segment (start 175.3 104.14) (end 175.3 99.06) (width 0.2) (layer "F.Cu") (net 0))
 (segment (start 167.64 106.405) (end 170.535 106.405) (width 0.2) (layer "F.Cu") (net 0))
 (segment (start 170.18 91.44) (end 172.72 88.9) (width 0.2) (layer "F.Cu") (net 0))
 (segment (start 175.3 109.22) (end 175.3 104.14) (width 0.2) (layer "F.Cu") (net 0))
 (segment (start 190.5 96.52) (end 187.96 93.98) (width 0.2) (layer "F.Cu") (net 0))
 (segment (start 187.96 93.98) (end 187.92 93.98) (width 0.2) (layer "F.Cu") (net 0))
 (segment (start 190.185 111.485) (end 187.92 109.22) (width 0.2) (layer "F.Cu") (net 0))
 (segment (start 175.26 81.28) (end 185.42 91.44) (width 0.2) (layer "F.Cu") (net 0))
 (segment (start 193.04 108.945) (end 188.235 104.14) (width 0.2) (layer "F.Cu") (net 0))
 (segment (start 167.64 98.785) (end 170.18 96.245) (width 0.2) (layer "F.Cu") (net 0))
 (segment (start 187.92 101.285) (end 187.92 99.06) (width 0.2) (layer "F.Cu") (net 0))
 (segment (start 193.04 114.025) (end 188.275 114.025) (width 0.2) (layer "F.Cu") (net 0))
 (segment (start 175.3 93.98) (end 175.3 88.9) (width 0.2) (layer "F.Cu") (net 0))
 (segment (start 193.04 111.485) (end 190.185 111.485) (width 0.2) (layer "F.Cu") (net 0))
 (segment (start 167.64 108.945) (end 172.525 108.945) (width 0.2) (layer "F.Cu") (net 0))
 (segment (start 175.3 99.06) (end 175.3 93.98) (width 0.2) (layer "F.Cu") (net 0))
 (segment (start 193.04 106.405) (end 187.92 101.285) (width 0.2) (layer "F.Cu") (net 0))
 (segment (start 167.64 81.28) (end 175.26 81.28) (width 0.2) (layer "F.Cu") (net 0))
 (segment (start 172.445 99.06) (end 172.8 99.06) (width 0.2) (layer "F.Cu") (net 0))
 (segment (start 172.525 108.945) (end 172.8 109.22) (width 0.2) (layer "F.Cu") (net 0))
 (segment (start 185.5 109.3) (end 185.42 109.22) (width 0.2) (layer "F.Cu") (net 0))
 (segment (start 183 109.3) (end 182.92 109.22) (width 0.2) (layer "B.Cu") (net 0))
 (segment (start 177.8 111.76) (end 177.8 109.22) (width 0.2) (layer "B.Cu") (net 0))
 (segment (start 182.92 104.14) (end 182.92 99.06) (width 0.2) (layer "B.Cu") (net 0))
 (segment (start 175.26 83.82) (end 167.64 83.82) (width 0.2) (layer "B.Cu") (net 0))
 (segment (start 175.26 114.3) (end 183 114.3) (width 0.2) (layer "B.Cu") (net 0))
 (segment (start 183 114.3) (end 183 109.3) (width 0.2) (layer "B.Cu") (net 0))
 (segment (start 177.8 109.22) (end 177.8 104.14) (width 0.2) (layer "B.Cu") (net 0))
 (segment (start 175.26 114.3) (end 177.8 111.76) (width 0.2) (layer "B.Cu") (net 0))
 (segment (start 182.92 109.22) (end 182.92 104.14) (width 0.2) (layer "B.Cu") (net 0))
 (segment (start 177.8 86.36) (end 175.26 83.82) (width 0.2) (layer "B.Cu") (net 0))
 (segment (start 177.8 99.06) (end 177.8 93.98) (width 0.2) (layer "B.Cu") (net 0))
 (segment (start 177.8 104.14) (end 177.8 99.06) (width 0.2) (layer "B.Cu") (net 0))
 (segment (start 177.8 88.9) (end 177.8 86.36) (width 0.2) (layer "B.Cu") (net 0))
 (segment (start 177.8 93.98) (end 177.8 88.9) (width 0.2) (layer "B.Cu") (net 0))
 (segment (start 182.92 99.06) (end 182.92 93.98) (width 0.2) (layer "B.Cu") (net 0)))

